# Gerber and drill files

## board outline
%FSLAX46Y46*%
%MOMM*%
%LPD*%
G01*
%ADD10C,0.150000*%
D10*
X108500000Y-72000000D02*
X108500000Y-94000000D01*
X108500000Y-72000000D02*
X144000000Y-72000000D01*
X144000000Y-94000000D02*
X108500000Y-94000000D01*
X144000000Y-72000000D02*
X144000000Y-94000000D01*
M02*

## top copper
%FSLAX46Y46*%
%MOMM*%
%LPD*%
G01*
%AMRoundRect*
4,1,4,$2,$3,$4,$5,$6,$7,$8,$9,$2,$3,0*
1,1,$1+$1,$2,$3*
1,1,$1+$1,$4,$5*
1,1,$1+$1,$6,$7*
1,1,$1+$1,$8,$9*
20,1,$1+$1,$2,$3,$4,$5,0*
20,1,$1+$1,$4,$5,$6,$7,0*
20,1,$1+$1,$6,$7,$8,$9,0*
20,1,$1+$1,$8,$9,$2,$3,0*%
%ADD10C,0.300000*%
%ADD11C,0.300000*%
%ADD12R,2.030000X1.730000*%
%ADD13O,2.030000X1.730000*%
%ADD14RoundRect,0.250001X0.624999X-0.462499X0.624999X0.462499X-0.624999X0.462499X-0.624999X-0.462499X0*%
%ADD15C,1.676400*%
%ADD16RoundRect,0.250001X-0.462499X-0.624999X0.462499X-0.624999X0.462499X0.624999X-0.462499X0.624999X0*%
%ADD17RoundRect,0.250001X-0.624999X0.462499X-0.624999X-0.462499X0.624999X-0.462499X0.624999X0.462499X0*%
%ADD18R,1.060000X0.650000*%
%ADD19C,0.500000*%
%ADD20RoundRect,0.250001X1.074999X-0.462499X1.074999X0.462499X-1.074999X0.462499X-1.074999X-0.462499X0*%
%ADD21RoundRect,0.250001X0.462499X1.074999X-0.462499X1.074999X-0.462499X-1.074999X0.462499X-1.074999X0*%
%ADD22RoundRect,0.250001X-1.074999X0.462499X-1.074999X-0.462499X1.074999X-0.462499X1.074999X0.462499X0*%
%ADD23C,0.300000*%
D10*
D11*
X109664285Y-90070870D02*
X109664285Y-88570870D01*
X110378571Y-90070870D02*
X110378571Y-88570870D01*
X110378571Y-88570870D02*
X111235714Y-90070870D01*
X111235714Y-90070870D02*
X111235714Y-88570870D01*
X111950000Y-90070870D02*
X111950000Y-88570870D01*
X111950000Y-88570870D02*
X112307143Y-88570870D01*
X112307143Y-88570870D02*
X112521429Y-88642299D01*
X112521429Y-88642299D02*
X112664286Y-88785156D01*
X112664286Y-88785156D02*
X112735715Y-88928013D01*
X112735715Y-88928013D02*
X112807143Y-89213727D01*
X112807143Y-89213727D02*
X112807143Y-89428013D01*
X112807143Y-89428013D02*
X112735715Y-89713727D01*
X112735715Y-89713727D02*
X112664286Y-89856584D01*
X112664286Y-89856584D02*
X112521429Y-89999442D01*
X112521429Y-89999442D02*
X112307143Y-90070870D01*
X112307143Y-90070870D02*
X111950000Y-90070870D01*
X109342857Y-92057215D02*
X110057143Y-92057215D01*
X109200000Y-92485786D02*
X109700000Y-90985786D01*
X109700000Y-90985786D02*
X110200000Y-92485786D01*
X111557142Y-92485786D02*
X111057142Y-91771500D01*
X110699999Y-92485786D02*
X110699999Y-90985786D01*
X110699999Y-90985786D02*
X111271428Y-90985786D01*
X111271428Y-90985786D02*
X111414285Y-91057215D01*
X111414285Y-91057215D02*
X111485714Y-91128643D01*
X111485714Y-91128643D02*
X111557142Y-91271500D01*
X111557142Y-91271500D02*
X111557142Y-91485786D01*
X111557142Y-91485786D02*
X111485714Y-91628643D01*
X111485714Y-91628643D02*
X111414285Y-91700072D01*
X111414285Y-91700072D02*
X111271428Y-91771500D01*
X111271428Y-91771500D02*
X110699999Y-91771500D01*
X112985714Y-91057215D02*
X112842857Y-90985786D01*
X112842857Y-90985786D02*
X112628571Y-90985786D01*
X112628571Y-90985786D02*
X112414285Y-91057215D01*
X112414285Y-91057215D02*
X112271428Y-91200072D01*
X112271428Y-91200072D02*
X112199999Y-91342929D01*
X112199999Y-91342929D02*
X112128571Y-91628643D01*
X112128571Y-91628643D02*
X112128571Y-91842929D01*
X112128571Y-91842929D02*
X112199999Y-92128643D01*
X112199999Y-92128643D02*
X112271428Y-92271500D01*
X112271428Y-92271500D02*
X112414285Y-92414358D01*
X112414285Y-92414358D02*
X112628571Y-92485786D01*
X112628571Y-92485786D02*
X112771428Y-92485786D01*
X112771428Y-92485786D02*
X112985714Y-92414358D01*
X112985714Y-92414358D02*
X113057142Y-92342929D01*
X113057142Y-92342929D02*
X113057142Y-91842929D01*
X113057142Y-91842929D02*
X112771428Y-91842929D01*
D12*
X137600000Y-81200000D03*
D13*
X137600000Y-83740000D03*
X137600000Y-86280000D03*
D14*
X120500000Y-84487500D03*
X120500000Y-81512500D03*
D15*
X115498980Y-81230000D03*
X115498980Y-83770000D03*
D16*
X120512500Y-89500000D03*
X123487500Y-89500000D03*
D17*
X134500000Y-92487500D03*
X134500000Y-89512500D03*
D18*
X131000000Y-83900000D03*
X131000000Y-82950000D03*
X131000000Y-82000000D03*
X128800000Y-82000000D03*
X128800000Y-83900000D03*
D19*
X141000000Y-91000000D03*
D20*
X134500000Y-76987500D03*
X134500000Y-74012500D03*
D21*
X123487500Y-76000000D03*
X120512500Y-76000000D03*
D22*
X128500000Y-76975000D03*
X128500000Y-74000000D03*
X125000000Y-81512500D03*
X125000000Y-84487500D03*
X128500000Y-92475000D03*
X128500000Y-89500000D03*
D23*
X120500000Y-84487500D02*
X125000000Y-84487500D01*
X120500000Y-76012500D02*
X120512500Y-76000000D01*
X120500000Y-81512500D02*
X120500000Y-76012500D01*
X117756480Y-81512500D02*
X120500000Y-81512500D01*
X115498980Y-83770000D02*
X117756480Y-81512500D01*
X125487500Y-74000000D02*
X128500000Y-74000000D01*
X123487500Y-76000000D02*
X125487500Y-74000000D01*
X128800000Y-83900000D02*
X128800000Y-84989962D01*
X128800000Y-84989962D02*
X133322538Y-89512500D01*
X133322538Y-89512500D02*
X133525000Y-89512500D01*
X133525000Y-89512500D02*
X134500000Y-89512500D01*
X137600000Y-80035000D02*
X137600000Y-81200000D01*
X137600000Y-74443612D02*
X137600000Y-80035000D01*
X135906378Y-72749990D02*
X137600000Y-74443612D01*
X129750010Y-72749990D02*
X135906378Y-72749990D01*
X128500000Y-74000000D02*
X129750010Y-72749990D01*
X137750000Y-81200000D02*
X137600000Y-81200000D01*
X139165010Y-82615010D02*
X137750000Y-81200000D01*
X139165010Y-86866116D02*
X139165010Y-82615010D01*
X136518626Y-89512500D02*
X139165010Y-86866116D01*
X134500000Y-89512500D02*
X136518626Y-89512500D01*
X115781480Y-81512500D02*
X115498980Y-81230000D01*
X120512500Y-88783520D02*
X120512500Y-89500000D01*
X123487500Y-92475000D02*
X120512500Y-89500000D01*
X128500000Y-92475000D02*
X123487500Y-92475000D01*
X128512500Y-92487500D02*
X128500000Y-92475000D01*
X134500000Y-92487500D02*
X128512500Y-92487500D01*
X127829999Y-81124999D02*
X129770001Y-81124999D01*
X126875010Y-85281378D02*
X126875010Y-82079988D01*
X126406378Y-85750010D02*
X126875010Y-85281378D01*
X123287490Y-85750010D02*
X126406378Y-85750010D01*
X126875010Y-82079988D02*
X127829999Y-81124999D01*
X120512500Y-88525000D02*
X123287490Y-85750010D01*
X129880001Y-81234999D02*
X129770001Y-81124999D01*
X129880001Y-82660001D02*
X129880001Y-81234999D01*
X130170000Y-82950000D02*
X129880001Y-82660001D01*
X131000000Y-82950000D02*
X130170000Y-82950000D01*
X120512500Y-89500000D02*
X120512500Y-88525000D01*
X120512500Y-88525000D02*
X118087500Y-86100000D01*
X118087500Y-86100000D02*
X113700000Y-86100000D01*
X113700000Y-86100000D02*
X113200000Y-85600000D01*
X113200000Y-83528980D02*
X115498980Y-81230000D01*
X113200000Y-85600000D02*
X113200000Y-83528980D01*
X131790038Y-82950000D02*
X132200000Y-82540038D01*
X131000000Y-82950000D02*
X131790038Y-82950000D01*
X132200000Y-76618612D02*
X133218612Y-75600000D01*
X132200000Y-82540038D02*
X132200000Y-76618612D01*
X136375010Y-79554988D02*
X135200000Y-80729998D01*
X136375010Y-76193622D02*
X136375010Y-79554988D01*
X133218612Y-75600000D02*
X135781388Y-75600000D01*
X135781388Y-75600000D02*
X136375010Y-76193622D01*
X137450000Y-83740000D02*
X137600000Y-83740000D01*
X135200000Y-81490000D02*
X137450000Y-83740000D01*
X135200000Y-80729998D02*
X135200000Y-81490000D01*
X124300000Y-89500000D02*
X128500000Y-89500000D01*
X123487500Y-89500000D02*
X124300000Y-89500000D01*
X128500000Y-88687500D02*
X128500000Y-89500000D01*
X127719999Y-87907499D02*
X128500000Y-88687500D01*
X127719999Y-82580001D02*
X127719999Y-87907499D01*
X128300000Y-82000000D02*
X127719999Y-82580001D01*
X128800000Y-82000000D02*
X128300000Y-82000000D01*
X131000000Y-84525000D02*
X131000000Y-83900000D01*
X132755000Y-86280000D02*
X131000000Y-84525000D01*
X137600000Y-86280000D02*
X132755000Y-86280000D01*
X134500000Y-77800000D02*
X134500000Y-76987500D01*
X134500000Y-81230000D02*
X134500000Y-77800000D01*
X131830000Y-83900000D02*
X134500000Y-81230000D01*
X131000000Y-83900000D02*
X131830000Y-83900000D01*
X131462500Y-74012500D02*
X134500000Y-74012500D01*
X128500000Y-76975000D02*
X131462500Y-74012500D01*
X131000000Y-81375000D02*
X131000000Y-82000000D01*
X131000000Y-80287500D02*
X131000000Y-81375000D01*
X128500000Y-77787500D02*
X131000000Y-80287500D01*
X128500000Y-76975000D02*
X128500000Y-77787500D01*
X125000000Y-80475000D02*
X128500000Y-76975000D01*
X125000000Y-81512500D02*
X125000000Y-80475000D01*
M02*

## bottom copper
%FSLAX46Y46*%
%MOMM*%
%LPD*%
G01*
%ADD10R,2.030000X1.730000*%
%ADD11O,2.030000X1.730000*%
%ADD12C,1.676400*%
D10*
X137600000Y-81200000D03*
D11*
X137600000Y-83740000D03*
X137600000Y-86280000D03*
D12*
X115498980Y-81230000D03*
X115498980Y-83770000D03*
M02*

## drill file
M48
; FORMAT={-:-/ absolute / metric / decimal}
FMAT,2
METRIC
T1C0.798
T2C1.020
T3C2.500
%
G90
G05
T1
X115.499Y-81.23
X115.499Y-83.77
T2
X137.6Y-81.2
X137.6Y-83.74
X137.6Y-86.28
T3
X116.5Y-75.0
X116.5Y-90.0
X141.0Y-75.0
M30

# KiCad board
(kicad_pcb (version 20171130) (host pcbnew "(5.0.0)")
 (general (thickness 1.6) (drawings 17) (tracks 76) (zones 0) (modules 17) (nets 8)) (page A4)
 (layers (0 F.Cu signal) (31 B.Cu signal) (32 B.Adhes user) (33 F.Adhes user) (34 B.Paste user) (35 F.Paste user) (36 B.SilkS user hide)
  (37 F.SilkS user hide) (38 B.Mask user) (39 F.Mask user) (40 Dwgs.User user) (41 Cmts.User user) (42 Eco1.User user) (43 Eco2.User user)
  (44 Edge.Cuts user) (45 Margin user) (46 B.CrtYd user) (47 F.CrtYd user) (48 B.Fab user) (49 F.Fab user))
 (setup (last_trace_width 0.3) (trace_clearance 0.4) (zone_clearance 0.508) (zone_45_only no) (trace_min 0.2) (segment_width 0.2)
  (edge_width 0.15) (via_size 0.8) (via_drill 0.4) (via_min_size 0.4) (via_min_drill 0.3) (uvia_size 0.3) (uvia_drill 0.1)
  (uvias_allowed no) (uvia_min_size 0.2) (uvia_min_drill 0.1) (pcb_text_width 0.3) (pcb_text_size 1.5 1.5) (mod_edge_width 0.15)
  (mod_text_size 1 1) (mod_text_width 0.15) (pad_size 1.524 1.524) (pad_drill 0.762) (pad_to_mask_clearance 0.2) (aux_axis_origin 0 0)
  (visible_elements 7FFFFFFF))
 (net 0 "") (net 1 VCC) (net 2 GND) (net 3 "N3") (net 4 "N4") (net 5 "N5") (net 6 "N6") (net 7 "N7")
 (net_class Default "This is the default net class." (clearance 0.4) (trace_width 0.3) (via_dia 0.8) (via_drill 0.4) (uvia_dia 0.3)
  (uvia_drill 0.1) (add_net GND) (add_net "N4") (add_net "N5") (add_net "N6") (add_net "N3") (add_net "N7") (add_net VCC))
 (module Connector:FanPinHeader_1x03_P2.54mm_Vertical (layer B.Cu) (at 137.6 81.2 270)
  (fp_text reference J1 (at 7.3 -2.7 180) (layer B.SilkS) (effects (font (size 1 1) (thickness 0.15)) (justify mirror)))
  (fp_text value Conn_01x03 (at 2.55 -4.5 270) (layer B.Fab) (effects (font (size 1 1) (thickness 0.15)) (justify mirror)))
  (pad 1 thru_hole rect (at 0 0 180) (size 2.03 1.73) (drill 1.02) (layers *.Cu *.Mask) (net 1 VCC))
  (pad 2 thru_hole oval (at 2.54 0 180) (size 2.03 1.73) (drill 1.02) (layers *.Cu *.Mask) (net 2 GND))
  (pad 3 thru_hole oval (at 5.08 0 180) (size 2.03 1.73) (drill 1.02) (layers *.Cu *.Mask) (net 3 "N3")))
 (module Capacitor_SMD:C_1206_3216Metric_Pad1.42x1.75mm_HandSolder (layer F.Cu) (at 120.5 83 90)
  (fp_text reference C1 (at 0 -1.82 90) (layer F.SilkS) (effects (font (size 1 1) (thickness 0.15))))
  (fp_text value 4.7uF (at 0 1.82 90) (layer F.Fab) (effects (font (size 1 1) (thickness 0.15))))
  (pad 1 smd roundrect (at -1.4875 0 90) (size 1.425 1.75) (layers F.Cu F.Paste F.Mask) (roundrect_rratio 0.175439) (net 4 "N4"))
  (pad 2 smd roundrect (at 1.4875 0 90) (size 1.425 1.75) (layers F.Cu F.Paste F.Mask) (roundrect_rratio 0.175439) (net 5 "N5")))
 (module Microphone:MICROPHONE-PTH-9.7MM (layer B.Cu) (at 113.5 82.5 180)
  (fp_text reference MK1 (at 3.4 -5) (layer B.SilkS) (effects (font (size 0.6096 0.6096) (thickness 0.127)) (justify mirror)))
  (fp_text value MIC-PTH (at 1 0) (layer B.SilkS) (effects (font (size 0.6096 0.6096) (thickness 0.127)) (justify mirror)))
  (pad OUT thru_hole circle (at -1.99898 1.27 180) (size 1.6764 1.6764) (drill 0.79756) (layers *.Cu *.Mask) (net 2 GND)
   (solder_mask_margin 0.1016))
  (pad GND thru_hole circle (at -1.99898 -1.27 180) (size 1.6764 1.6764) (drill 0.79756) (layers *.Cu *.Mask) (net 5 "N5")
   (solder_mask_margin 0.1016)))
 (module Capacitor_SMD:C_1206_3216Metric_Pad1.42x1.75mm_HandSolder (layer F.Cu) (at 122 89.5)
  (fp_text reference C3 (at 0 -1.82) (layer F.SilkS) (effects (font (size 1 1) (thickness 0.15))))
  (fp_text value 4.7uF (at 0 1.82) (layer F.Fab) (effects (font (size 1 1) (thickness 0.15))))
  (pad 1 smd roundrect (at -1.4875 0) (size 1.425 1.75) (layers F.Cu F.Paste F.Mask) (roundrect_rratio 0.175439) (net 2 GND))
  (pad 2 smd roundrect (at 1.4875 0) (size 1.425 1.75) (layers F.Cu F.Paste F.Mask) (roundrect_rratio 0.175439) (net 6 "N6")))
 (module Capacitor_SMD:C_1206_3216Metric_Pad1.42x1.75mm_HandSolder (layer F.Cu) (at 134.5 91 270)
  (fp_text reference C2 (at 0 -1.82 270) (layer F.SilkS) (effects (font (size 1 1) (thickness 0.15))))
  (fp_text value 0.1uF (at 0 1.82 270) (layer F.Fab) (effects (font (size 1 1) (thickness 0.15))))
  (pad 2 smd roundrect (at 1.4875 0 270) (size 1.425 1.75) (layers F.Cu F.Paste F.Mask) (roundrect_rratio 0.175439) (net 2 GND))
  (pad 1 smd roundrect (at -1.4875 0 270) (size 1.425 1.75) (layers F.Cu F.Paste F.Mask) (roundrect_rratio 0.175439) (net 1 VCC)))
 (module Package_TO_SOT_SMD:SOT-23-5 (layer F.Cu) (at 129.9 82.95 180) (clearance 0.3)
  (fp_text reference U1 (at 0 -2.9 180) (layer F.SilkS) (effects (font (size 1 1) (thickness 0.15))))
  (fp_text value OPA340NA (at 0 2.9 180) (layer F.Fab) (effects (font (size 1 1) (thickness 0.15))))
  (pad 1 smd rect (at -1.1 -0.95 180) (size 1.06 0.65) (layers F.Cu F.Paste F.Mask) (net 3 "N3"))
  (pad 2 smd rect (at -1.1 0 180) (size 1.06 0.65) (layers F.Cu F.Paste F.Mask) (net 2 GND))
  (pad 3 smd rect (at -1.1 0.95 180) (size 1.06 0.65) (layers F.Cu F.Paste F.Mask) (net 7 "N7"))
  (pad 4 smd rect (at 1.1 0.95 180) (size 1.06 0.65) (layers F.Cu F.Paste F.Mask) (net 6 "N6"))
  (pad 5 smd rect (at 1.1 -0.95 180) (size 1.06 0.65) (layers F.Cu F.Paste F.Mask) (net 1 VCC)))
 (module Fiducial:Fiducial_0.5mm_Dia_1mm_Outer (layer F.Cu) (at 141 91)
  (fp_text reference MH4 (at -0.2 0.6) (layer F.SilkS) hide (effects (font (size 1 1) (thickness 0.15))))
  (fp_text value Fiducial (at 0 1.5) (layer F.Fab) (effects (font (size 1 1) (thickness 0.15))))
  (pad ~ smd circle (at 0 0) (size 0.5 0.5) (layers F.Cu F.Mask) (solder_mask_margin 0.25) (clearance 0.25)))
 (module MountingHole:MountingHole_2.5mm (layer F.Cu) (at 141 75)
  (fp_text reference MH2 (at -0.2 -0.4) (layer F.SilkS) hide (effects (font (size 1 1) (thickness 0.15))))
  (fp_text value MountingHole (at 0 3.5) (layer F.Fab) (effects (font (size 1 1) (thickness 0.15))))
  (pad 1 np_thru_hole circle (at 0 0) (size 2.5 2.5) (drill 2.5) (layers *.Cu *.Mask)))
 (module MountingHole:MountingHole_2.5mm (layer F.Cu) (at 116.5 90)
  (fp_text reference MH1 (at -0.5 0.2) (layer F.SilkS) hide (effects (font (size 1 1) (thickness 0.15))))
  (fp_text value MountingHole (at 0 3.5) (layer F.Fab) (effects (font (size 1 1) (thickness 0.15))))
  (pad 1 np_thru_hole circle (at 0 0) (size 2.5 2.5) (drill 2.5) (layers *.Cu *.Mask)))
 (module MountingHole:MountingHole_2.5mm (layer F.Cu) (at 116.5 75)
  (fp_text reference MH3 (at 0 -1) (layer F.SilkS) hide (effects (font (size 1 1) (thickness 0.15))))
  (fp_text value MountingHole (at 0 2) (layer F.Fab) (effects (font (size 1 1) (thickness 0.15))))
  (pad 1 np_thru_hole circle (at 0 0) (size 2.5 2.5) (drill 2.5) (layers *.Cu *.Mask)))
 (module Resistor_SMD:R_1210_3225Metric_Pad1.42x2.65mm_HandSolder (layer F.Cu) (at 134.5 75.5 90)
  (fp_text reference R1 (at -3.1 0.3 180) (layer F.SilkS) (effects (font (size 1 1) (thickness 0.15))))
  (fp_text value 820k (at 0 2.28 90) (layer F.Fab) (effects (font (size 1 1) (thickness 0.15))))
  (pad 1 smd roundrect (at -1.4875 0 90) (size 1.425 2.65) (layers F.Cu F.Paste F.Mask) (roundrect_rratio 0.175439) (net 3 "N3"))
  (pad 2 smd roundrect (at 1.4875 0 90) (size 1.425 2.65) (layers F.Cu F.Paste F.Mask) (roundrect_rratio 0.175439) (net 7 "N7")))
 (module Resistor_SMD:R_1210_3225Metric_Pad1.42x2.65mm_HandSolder (layer F.Cu) (at 122 76 180)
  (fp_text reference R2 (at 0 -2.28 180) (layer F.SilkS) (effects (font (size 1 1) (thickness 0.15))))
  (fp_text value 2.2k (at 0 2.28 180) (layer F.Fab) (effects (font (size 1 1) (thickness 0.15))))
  (pad 1 smd roundrect (at -1.4875 0 180) (size 1.425 2.65) (layers F.Cu F.Paste F.Mask) (roundrect_rratio 0.175439) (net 1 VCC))
  (pad 2 smd roundrect (at 1.4875 0 180) (size 1.425 2.65) (layers F.Cu F.Paste F.Mask) (roundrect_rratio 0.175439) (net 5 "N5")))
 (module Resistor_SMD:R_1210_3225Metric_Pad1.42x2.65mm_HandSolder (layer F.Cu) (at 128.5 75.4875 270)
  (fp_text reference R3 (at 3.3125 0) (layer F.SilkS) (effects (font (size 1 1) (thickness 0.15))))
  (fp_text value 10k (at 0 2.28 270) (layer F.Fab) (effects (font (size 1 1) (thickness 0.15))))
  (pad 2 smd roundrect (at 1.4875 0 270) (size 1.425 2.65) (layers F.Cu F.Paste F.Mask) (roundrect_rratio 0.175439) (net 7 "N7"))
  (pad 1 smd roundrect (at -1.4875 0 270) (size 1.425 2.65) (layers F.Cu F.Paste F.Mask) (roundrect_rratio 0.175439) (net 1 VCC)))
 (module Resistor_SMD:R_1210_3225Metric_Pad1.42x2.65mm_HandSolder (layer F.Cu) (at 125 83 270)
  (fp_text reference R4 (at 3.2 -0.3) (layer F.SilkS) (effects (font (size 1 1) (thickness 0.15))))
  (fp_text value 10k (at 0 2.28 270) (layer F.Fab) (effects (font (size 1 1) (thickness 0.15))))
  (pad 1 smd roundrect (at -1.4875 0 270) (size 1.425 2.65) (layers F.Cu F.Paste F.Mask) (roundrect_rratio 0.175439) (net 7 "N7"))
  (pad 2 smd roundrect (at 1.4875 0 270) (size 1.425 2.65) (layers F.Cu F.Paste F.Mask) (roundrect_rratio 0.175439) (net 4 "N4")))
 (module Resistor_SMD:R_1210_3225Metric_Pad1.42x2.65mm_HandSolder (layer F.Cu) (at 128.5 90.9875 270)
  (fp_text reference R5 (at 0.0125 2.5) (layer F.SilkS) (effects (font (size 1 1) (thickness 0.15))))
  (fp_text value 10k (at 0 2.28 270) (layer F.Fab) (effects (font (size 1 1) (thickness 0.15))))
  (pad 2 smd roundrect (at 1.4875 0 270) (size 1.425 2.65) (layers F.Cu F.Paste F.Mask) (roundrect_rratio 0.175439) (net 2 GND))
  (pad 1 smd roundrect (at -1.4875 0 270) (size 1.425 2.65) (layers F.Cu F.Paste F.Mask) (roundrect_rratio 0.175439) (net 6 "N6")))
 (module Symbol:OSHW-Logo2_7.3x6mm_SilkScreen (layer F.Cu) (at 112.2 77.5)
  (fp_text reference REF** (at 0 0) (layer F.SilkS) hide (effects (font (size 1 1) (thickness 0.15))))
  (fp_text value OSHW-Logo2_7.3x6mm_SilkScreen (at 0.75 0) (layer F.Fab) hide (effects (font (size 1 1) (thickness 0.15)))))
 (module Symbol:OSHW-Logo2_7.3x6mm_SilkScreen (layer B.Cu) (at 123.1 83.1 180)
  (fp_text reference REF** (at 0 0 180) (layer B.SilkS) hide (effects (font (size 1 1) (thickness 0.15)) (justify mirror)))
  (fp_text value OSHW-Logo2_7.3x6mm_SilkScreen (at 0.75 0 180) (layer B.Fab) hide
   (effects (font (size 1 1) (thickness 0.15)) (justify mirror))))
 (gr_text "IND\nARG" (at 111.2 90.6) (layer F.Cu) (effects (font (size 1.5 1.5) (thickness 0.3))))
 (gr_line (start 108.5 72) (end 108.5 94) (layer Edge.Cuts) (width 0.15))
 (gr_line (start 108.5 72) (end 144 72) (layer Edge.Cuts) (width 0.15))
 (gr_line (start 144 94) (end 108.5 94) (layer Edge.Cuts) (width 0.15))
 (gr_line (start 144 72) (end 144 94) (layer Edge.Cuts) (width 0.15))
 (segment (start 120.5 84.4875) (end 125 84.4875) (width 0.3) (layer F.Cu) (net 4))
 (segment (start 120.5 76.0125) (end 120.5125 76) (width 0.3) (layer F.Cu) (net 5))
 (segment (start 120.5 81.5125) (end 120.5 76.0125) (width 0.3) (layer F.Cu) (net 5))
 (segment (start 117.75648 81.5125) (end 120.5 81.5125) (width 0.3) (layer F.Cu) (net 5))
 (segment (start 115.49898 83.77) (end 117.75648 81.5125) (width 0.3) (layer F.Cu) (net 5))
 (segment (start 125.4875 74) (end 128.5 74) (width 0.3) (layer F.Cu) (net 1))
 (segment (start 123.4875 76) (end 125.4875 74) (width 0.3) (layer F.Cu) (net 1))
 (segment (start 128.8 83.9) (end 128.8 84.989962) (width 0.3) (layer F.Cu) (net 1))
 (segment (start 128.8 84.989962) (end 133.322538 89.5125) (width 0.3) (layer F.Cu) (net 1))
 (segment (start 133.322538 89.5125) (end 133.525 89.5125) (width 0.3) (layer F.Cu) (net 1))
 (segment (start 133.525 89.5125) (end 134.5 89.5125) (width 0.3) (layer F.Cu) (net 1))
 (segment (start 137.6 80.035) (end 137.6 81.2) (width 0.3) (layer F.Cu) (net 1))
 (segment (start 137.6 74.443612) (end 137.6 80.035) (width 0.3) (layer F.Cu) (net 1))
 (segment (start 135.906378 72.74999) (end 137.6 74.443612) (width 0.3) (layer F.Cu) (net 1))
 (segment (start 129.75001 72.74999) (end 135.906378 72.74999) (width 0.3) (layer F.Cu) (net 1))
 (segment (start 128.5 74) (end 129.75001 72.74999) (width 0.3) (layer F.Cu) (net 1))
 (segment (start 137.75 81.2) (end 137.6 81.2) (width 0.3) (layer F.Cu) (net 1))
 (segment (start 139.16501 82.61501) (end 137.75 81.2) (width 0.3) (layer F.Cu) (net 1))
 (segment (start 139.16501 86.866116) (end 139.16501 82.61501) (width 0.3) (layer F.Cu) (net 1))
 (segment (start 136.518626 89.5125) (end 139.16501 86.866116) (width 0.3) (layer F.Cu) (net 1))
 (segment (start 134.5 89.5125) (end 136.518626 89.5125) (width 0.3) (layer F.Cu) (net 1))
 (segment (start 115.78148 81.5125) (end 115.49898 81.23) (width 0.3) (layer F.Cu) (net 2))
 (segment (start 120.5125 88.78352) (end 120.5125 89.5) (width 0.3) (layer F.Cu) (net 2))
 (segment (start 123.4875 92.475) (end 120.5125 89.5) (width 0.3) (layer F.Cu) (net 2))
 (segment (start 128.5 92.475) (end 123.4875 92.475) (width 0.3) (layer F.Cu) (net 2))
 (segment (start 128.5125 92.4875) (end 128.5 92.475) (width 0.3) (layer F.Cu) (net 2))
 (segment (start 134.5 92.4875) (end 128.5125 92.4875) (width 0.3) (layer F.Cu) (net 2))
 (segment (start 127.829999 81.124999) (end 129.770001 81.124999) (width 0.3) (layer F.Cu) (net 2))
 (segment (start 126.87501 85.281378) (end 126.87501 82.079988) (width 0.3) (layer F.Cu) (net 2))
 (segment (start 126.406378 85.75001) (end 126.87501 85.281378) (width 0.3) (layer F.Cu) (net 2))
 (segment (start 123.28749 85.75001) (end 126.406378 85.75001) (width 0.3) (layer F.Cu) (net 2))
 (segment (start 126.87501 82.079988) (end 127.829999 81.124999) (width 0.3) (layer F.Cu) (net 2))
 (segment (start 120.5125 88.525) (end 123.28749 85.75001) (width 0.3) (layer F.Cu) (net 2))
 (segment (start 129.880001 81.234999) (end 129.770001 81.124999) (width 0.3) (layer F.Cu) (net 2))
 (segment (start 129.880001 82.660001) (end 129.880001 81.234999) (width 0.3) (layer F.Cu) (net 2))
 (segment (start 130.17 82.95) (end 129.880001 82.660001) (width 0.3) (layer F.Cu) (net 2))
 (segment (start 131 82.95) (end 130.17 82.95) (width 0.3) (layer F.Cu) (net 2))
 (segment (start 120.5125 89.5) (end 120.5125 88.525) (width 0.3) (layer F.Cu) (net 2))
 (segment (start 120.5125 88.525) (end 118.0875 86.1) (width 0.3) (layer F.Cu) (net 2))
 (segment (start 118.0875 86.1) (end 113.7 86.1) (width 0.3) (layer F.Cu) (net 2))
 (segment (start 113.7 86.1) (end 113.2 85.6) (width 0.3) (layer F.Cu) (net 2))
 (segment (start 113.2 83.52898) (end 115.49898 81.23) (width 0.3) (layer F.Cu) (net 2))
 (segment (start 113.2 85.6) (end 113.2 83.52898) (width 0.3) (layer F.Cu) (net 2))
 (segment (start 131.790038 82.95) (end 132.2 82.540038) (width 0.3) (layer F.Cu) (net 2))
 (segment (start 131 82.95) (end 131.790038 82.95) (width 0.3) (layer F.Cu) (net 2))
 (segment (start 132.2 76.618612) (end 133.218612 75.6) (width 0.3) (layer F.Cu) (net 2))
 (segment (start 132.2 82.540038) (end 132.2 76.618612) (width 0.3) (layer F.Cu) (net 2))
 (segment (start 136.37501 79.554988) (end 135.2 80.729998) (width 0.3) (layer F.Cu) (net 2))
 (segment (start 136.37501 76.193622) (end 136.37501 79.554988) (width 0.3) (layer F.Cu) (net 2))
 (segment (start 133.218612 75.6) (end 135.781388 75.6) (width 0.3) (layer F.Cu) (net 2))
 (segment (start 135.781388 75.6) (end 136.37501 76.193622) (width 0.3) (layer F.Cu) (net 2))
 (segment (start 137.45 83.74) (end 137.6 83.74) (width 0.3) (layer F.Cu) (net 2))
 (segment (start 135.2 81.49) (end 137.45 83.74) (width 0.3) (layer F.Cu) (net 2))
 (segment (start 135.2 80.729998) (end 135.2 81.49) (width 0.3) (layer F.Cu) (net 2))
 (segment (start 124.3 89.5) (end 128.5 89.5) (width 0.3) (layer F.Cu) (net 6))
 (segment (start 123.4875 89.5) (end 124.3 89.5) (width 0.3) (layer F.Cu) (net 6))
 (segment (start 128.5 88.6875) (end 128.5 89.5) (width 0.3) (layer F.Cu) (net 6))
 (segment (start 127.719999 87.907499) (end 128.5 88.6875) (width 0.3) (layer F.Cu) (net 6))
 (segment (start 127.719999 82.580001) (end 127.719999 87.907499) (width 0.3) (layer F.Cu) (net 6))
 (segment (start 128.3 82) (end 127.719999 82.580001) (width 0.3) (layer F.Cu) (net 6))
 (segment (start 128.8 82) (end 128.3 82) (width 0.3) (layer F.Cu) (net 6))
 (segment (start 131 84.525) (end 131 83.9) (width 0.3) (layer F.Cu) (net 3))
 (segment (start 132.755 86.28) (end 131 84.525) (width 0.3) (layer F.Cu) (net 3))
 (segment (start 137.6 86.28) (end 132.755 86.28) (width 0.3) (layer F.Cu) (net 3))
 (segment (start 134.5 77.8) (end 134.5 76.9875) (width 0.3) (layer F.Cu) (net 3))
 (segment (start 134.5 81.23) (end 134.5 77.8) (width 0.3) (layer F.Cu) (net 3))
 (segment (start 131.83 83.9) (end 134.5 81.23) (width 0.3) (layer F.Cu) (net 3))
 (segment (start 131 83.9) (end 131.83 83.9) (width 0.3) (layer F.Cu) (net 3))
 (segment (start 131.4625 74.0125) (end 134.5 74.0125) (width 0.3) (layer F.Cu) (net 7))
 (segment (start 128.5 76.975) (end 131.4625 74.0125) (width 0.3) (layer F.Cu) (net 7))
 (segment (start 131 81.375) (end 131 82) (width 0.3) (layer F.Cu) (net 7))
 (segment (start 131 80.2875) (end 131 81.375) (width 0.3) (layer F.Cu) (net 7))
 (segment (start 128.5 77.7875) (end 131 80.2875) (width 0.3) (layer F.Cu) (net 7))
 (segment (start 128.5 76.975) (end 128.5 77.7875) (width 0.3) (layer F.Cu) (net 7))
 (segment (start 125 80.475) (end 128.5 76.975) (width 0.3) (layer F.Cu) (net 7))
 (segment (start 125 81.5125) (end 125 80.475) (width 0.3) (layer F.Cu) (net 7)))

